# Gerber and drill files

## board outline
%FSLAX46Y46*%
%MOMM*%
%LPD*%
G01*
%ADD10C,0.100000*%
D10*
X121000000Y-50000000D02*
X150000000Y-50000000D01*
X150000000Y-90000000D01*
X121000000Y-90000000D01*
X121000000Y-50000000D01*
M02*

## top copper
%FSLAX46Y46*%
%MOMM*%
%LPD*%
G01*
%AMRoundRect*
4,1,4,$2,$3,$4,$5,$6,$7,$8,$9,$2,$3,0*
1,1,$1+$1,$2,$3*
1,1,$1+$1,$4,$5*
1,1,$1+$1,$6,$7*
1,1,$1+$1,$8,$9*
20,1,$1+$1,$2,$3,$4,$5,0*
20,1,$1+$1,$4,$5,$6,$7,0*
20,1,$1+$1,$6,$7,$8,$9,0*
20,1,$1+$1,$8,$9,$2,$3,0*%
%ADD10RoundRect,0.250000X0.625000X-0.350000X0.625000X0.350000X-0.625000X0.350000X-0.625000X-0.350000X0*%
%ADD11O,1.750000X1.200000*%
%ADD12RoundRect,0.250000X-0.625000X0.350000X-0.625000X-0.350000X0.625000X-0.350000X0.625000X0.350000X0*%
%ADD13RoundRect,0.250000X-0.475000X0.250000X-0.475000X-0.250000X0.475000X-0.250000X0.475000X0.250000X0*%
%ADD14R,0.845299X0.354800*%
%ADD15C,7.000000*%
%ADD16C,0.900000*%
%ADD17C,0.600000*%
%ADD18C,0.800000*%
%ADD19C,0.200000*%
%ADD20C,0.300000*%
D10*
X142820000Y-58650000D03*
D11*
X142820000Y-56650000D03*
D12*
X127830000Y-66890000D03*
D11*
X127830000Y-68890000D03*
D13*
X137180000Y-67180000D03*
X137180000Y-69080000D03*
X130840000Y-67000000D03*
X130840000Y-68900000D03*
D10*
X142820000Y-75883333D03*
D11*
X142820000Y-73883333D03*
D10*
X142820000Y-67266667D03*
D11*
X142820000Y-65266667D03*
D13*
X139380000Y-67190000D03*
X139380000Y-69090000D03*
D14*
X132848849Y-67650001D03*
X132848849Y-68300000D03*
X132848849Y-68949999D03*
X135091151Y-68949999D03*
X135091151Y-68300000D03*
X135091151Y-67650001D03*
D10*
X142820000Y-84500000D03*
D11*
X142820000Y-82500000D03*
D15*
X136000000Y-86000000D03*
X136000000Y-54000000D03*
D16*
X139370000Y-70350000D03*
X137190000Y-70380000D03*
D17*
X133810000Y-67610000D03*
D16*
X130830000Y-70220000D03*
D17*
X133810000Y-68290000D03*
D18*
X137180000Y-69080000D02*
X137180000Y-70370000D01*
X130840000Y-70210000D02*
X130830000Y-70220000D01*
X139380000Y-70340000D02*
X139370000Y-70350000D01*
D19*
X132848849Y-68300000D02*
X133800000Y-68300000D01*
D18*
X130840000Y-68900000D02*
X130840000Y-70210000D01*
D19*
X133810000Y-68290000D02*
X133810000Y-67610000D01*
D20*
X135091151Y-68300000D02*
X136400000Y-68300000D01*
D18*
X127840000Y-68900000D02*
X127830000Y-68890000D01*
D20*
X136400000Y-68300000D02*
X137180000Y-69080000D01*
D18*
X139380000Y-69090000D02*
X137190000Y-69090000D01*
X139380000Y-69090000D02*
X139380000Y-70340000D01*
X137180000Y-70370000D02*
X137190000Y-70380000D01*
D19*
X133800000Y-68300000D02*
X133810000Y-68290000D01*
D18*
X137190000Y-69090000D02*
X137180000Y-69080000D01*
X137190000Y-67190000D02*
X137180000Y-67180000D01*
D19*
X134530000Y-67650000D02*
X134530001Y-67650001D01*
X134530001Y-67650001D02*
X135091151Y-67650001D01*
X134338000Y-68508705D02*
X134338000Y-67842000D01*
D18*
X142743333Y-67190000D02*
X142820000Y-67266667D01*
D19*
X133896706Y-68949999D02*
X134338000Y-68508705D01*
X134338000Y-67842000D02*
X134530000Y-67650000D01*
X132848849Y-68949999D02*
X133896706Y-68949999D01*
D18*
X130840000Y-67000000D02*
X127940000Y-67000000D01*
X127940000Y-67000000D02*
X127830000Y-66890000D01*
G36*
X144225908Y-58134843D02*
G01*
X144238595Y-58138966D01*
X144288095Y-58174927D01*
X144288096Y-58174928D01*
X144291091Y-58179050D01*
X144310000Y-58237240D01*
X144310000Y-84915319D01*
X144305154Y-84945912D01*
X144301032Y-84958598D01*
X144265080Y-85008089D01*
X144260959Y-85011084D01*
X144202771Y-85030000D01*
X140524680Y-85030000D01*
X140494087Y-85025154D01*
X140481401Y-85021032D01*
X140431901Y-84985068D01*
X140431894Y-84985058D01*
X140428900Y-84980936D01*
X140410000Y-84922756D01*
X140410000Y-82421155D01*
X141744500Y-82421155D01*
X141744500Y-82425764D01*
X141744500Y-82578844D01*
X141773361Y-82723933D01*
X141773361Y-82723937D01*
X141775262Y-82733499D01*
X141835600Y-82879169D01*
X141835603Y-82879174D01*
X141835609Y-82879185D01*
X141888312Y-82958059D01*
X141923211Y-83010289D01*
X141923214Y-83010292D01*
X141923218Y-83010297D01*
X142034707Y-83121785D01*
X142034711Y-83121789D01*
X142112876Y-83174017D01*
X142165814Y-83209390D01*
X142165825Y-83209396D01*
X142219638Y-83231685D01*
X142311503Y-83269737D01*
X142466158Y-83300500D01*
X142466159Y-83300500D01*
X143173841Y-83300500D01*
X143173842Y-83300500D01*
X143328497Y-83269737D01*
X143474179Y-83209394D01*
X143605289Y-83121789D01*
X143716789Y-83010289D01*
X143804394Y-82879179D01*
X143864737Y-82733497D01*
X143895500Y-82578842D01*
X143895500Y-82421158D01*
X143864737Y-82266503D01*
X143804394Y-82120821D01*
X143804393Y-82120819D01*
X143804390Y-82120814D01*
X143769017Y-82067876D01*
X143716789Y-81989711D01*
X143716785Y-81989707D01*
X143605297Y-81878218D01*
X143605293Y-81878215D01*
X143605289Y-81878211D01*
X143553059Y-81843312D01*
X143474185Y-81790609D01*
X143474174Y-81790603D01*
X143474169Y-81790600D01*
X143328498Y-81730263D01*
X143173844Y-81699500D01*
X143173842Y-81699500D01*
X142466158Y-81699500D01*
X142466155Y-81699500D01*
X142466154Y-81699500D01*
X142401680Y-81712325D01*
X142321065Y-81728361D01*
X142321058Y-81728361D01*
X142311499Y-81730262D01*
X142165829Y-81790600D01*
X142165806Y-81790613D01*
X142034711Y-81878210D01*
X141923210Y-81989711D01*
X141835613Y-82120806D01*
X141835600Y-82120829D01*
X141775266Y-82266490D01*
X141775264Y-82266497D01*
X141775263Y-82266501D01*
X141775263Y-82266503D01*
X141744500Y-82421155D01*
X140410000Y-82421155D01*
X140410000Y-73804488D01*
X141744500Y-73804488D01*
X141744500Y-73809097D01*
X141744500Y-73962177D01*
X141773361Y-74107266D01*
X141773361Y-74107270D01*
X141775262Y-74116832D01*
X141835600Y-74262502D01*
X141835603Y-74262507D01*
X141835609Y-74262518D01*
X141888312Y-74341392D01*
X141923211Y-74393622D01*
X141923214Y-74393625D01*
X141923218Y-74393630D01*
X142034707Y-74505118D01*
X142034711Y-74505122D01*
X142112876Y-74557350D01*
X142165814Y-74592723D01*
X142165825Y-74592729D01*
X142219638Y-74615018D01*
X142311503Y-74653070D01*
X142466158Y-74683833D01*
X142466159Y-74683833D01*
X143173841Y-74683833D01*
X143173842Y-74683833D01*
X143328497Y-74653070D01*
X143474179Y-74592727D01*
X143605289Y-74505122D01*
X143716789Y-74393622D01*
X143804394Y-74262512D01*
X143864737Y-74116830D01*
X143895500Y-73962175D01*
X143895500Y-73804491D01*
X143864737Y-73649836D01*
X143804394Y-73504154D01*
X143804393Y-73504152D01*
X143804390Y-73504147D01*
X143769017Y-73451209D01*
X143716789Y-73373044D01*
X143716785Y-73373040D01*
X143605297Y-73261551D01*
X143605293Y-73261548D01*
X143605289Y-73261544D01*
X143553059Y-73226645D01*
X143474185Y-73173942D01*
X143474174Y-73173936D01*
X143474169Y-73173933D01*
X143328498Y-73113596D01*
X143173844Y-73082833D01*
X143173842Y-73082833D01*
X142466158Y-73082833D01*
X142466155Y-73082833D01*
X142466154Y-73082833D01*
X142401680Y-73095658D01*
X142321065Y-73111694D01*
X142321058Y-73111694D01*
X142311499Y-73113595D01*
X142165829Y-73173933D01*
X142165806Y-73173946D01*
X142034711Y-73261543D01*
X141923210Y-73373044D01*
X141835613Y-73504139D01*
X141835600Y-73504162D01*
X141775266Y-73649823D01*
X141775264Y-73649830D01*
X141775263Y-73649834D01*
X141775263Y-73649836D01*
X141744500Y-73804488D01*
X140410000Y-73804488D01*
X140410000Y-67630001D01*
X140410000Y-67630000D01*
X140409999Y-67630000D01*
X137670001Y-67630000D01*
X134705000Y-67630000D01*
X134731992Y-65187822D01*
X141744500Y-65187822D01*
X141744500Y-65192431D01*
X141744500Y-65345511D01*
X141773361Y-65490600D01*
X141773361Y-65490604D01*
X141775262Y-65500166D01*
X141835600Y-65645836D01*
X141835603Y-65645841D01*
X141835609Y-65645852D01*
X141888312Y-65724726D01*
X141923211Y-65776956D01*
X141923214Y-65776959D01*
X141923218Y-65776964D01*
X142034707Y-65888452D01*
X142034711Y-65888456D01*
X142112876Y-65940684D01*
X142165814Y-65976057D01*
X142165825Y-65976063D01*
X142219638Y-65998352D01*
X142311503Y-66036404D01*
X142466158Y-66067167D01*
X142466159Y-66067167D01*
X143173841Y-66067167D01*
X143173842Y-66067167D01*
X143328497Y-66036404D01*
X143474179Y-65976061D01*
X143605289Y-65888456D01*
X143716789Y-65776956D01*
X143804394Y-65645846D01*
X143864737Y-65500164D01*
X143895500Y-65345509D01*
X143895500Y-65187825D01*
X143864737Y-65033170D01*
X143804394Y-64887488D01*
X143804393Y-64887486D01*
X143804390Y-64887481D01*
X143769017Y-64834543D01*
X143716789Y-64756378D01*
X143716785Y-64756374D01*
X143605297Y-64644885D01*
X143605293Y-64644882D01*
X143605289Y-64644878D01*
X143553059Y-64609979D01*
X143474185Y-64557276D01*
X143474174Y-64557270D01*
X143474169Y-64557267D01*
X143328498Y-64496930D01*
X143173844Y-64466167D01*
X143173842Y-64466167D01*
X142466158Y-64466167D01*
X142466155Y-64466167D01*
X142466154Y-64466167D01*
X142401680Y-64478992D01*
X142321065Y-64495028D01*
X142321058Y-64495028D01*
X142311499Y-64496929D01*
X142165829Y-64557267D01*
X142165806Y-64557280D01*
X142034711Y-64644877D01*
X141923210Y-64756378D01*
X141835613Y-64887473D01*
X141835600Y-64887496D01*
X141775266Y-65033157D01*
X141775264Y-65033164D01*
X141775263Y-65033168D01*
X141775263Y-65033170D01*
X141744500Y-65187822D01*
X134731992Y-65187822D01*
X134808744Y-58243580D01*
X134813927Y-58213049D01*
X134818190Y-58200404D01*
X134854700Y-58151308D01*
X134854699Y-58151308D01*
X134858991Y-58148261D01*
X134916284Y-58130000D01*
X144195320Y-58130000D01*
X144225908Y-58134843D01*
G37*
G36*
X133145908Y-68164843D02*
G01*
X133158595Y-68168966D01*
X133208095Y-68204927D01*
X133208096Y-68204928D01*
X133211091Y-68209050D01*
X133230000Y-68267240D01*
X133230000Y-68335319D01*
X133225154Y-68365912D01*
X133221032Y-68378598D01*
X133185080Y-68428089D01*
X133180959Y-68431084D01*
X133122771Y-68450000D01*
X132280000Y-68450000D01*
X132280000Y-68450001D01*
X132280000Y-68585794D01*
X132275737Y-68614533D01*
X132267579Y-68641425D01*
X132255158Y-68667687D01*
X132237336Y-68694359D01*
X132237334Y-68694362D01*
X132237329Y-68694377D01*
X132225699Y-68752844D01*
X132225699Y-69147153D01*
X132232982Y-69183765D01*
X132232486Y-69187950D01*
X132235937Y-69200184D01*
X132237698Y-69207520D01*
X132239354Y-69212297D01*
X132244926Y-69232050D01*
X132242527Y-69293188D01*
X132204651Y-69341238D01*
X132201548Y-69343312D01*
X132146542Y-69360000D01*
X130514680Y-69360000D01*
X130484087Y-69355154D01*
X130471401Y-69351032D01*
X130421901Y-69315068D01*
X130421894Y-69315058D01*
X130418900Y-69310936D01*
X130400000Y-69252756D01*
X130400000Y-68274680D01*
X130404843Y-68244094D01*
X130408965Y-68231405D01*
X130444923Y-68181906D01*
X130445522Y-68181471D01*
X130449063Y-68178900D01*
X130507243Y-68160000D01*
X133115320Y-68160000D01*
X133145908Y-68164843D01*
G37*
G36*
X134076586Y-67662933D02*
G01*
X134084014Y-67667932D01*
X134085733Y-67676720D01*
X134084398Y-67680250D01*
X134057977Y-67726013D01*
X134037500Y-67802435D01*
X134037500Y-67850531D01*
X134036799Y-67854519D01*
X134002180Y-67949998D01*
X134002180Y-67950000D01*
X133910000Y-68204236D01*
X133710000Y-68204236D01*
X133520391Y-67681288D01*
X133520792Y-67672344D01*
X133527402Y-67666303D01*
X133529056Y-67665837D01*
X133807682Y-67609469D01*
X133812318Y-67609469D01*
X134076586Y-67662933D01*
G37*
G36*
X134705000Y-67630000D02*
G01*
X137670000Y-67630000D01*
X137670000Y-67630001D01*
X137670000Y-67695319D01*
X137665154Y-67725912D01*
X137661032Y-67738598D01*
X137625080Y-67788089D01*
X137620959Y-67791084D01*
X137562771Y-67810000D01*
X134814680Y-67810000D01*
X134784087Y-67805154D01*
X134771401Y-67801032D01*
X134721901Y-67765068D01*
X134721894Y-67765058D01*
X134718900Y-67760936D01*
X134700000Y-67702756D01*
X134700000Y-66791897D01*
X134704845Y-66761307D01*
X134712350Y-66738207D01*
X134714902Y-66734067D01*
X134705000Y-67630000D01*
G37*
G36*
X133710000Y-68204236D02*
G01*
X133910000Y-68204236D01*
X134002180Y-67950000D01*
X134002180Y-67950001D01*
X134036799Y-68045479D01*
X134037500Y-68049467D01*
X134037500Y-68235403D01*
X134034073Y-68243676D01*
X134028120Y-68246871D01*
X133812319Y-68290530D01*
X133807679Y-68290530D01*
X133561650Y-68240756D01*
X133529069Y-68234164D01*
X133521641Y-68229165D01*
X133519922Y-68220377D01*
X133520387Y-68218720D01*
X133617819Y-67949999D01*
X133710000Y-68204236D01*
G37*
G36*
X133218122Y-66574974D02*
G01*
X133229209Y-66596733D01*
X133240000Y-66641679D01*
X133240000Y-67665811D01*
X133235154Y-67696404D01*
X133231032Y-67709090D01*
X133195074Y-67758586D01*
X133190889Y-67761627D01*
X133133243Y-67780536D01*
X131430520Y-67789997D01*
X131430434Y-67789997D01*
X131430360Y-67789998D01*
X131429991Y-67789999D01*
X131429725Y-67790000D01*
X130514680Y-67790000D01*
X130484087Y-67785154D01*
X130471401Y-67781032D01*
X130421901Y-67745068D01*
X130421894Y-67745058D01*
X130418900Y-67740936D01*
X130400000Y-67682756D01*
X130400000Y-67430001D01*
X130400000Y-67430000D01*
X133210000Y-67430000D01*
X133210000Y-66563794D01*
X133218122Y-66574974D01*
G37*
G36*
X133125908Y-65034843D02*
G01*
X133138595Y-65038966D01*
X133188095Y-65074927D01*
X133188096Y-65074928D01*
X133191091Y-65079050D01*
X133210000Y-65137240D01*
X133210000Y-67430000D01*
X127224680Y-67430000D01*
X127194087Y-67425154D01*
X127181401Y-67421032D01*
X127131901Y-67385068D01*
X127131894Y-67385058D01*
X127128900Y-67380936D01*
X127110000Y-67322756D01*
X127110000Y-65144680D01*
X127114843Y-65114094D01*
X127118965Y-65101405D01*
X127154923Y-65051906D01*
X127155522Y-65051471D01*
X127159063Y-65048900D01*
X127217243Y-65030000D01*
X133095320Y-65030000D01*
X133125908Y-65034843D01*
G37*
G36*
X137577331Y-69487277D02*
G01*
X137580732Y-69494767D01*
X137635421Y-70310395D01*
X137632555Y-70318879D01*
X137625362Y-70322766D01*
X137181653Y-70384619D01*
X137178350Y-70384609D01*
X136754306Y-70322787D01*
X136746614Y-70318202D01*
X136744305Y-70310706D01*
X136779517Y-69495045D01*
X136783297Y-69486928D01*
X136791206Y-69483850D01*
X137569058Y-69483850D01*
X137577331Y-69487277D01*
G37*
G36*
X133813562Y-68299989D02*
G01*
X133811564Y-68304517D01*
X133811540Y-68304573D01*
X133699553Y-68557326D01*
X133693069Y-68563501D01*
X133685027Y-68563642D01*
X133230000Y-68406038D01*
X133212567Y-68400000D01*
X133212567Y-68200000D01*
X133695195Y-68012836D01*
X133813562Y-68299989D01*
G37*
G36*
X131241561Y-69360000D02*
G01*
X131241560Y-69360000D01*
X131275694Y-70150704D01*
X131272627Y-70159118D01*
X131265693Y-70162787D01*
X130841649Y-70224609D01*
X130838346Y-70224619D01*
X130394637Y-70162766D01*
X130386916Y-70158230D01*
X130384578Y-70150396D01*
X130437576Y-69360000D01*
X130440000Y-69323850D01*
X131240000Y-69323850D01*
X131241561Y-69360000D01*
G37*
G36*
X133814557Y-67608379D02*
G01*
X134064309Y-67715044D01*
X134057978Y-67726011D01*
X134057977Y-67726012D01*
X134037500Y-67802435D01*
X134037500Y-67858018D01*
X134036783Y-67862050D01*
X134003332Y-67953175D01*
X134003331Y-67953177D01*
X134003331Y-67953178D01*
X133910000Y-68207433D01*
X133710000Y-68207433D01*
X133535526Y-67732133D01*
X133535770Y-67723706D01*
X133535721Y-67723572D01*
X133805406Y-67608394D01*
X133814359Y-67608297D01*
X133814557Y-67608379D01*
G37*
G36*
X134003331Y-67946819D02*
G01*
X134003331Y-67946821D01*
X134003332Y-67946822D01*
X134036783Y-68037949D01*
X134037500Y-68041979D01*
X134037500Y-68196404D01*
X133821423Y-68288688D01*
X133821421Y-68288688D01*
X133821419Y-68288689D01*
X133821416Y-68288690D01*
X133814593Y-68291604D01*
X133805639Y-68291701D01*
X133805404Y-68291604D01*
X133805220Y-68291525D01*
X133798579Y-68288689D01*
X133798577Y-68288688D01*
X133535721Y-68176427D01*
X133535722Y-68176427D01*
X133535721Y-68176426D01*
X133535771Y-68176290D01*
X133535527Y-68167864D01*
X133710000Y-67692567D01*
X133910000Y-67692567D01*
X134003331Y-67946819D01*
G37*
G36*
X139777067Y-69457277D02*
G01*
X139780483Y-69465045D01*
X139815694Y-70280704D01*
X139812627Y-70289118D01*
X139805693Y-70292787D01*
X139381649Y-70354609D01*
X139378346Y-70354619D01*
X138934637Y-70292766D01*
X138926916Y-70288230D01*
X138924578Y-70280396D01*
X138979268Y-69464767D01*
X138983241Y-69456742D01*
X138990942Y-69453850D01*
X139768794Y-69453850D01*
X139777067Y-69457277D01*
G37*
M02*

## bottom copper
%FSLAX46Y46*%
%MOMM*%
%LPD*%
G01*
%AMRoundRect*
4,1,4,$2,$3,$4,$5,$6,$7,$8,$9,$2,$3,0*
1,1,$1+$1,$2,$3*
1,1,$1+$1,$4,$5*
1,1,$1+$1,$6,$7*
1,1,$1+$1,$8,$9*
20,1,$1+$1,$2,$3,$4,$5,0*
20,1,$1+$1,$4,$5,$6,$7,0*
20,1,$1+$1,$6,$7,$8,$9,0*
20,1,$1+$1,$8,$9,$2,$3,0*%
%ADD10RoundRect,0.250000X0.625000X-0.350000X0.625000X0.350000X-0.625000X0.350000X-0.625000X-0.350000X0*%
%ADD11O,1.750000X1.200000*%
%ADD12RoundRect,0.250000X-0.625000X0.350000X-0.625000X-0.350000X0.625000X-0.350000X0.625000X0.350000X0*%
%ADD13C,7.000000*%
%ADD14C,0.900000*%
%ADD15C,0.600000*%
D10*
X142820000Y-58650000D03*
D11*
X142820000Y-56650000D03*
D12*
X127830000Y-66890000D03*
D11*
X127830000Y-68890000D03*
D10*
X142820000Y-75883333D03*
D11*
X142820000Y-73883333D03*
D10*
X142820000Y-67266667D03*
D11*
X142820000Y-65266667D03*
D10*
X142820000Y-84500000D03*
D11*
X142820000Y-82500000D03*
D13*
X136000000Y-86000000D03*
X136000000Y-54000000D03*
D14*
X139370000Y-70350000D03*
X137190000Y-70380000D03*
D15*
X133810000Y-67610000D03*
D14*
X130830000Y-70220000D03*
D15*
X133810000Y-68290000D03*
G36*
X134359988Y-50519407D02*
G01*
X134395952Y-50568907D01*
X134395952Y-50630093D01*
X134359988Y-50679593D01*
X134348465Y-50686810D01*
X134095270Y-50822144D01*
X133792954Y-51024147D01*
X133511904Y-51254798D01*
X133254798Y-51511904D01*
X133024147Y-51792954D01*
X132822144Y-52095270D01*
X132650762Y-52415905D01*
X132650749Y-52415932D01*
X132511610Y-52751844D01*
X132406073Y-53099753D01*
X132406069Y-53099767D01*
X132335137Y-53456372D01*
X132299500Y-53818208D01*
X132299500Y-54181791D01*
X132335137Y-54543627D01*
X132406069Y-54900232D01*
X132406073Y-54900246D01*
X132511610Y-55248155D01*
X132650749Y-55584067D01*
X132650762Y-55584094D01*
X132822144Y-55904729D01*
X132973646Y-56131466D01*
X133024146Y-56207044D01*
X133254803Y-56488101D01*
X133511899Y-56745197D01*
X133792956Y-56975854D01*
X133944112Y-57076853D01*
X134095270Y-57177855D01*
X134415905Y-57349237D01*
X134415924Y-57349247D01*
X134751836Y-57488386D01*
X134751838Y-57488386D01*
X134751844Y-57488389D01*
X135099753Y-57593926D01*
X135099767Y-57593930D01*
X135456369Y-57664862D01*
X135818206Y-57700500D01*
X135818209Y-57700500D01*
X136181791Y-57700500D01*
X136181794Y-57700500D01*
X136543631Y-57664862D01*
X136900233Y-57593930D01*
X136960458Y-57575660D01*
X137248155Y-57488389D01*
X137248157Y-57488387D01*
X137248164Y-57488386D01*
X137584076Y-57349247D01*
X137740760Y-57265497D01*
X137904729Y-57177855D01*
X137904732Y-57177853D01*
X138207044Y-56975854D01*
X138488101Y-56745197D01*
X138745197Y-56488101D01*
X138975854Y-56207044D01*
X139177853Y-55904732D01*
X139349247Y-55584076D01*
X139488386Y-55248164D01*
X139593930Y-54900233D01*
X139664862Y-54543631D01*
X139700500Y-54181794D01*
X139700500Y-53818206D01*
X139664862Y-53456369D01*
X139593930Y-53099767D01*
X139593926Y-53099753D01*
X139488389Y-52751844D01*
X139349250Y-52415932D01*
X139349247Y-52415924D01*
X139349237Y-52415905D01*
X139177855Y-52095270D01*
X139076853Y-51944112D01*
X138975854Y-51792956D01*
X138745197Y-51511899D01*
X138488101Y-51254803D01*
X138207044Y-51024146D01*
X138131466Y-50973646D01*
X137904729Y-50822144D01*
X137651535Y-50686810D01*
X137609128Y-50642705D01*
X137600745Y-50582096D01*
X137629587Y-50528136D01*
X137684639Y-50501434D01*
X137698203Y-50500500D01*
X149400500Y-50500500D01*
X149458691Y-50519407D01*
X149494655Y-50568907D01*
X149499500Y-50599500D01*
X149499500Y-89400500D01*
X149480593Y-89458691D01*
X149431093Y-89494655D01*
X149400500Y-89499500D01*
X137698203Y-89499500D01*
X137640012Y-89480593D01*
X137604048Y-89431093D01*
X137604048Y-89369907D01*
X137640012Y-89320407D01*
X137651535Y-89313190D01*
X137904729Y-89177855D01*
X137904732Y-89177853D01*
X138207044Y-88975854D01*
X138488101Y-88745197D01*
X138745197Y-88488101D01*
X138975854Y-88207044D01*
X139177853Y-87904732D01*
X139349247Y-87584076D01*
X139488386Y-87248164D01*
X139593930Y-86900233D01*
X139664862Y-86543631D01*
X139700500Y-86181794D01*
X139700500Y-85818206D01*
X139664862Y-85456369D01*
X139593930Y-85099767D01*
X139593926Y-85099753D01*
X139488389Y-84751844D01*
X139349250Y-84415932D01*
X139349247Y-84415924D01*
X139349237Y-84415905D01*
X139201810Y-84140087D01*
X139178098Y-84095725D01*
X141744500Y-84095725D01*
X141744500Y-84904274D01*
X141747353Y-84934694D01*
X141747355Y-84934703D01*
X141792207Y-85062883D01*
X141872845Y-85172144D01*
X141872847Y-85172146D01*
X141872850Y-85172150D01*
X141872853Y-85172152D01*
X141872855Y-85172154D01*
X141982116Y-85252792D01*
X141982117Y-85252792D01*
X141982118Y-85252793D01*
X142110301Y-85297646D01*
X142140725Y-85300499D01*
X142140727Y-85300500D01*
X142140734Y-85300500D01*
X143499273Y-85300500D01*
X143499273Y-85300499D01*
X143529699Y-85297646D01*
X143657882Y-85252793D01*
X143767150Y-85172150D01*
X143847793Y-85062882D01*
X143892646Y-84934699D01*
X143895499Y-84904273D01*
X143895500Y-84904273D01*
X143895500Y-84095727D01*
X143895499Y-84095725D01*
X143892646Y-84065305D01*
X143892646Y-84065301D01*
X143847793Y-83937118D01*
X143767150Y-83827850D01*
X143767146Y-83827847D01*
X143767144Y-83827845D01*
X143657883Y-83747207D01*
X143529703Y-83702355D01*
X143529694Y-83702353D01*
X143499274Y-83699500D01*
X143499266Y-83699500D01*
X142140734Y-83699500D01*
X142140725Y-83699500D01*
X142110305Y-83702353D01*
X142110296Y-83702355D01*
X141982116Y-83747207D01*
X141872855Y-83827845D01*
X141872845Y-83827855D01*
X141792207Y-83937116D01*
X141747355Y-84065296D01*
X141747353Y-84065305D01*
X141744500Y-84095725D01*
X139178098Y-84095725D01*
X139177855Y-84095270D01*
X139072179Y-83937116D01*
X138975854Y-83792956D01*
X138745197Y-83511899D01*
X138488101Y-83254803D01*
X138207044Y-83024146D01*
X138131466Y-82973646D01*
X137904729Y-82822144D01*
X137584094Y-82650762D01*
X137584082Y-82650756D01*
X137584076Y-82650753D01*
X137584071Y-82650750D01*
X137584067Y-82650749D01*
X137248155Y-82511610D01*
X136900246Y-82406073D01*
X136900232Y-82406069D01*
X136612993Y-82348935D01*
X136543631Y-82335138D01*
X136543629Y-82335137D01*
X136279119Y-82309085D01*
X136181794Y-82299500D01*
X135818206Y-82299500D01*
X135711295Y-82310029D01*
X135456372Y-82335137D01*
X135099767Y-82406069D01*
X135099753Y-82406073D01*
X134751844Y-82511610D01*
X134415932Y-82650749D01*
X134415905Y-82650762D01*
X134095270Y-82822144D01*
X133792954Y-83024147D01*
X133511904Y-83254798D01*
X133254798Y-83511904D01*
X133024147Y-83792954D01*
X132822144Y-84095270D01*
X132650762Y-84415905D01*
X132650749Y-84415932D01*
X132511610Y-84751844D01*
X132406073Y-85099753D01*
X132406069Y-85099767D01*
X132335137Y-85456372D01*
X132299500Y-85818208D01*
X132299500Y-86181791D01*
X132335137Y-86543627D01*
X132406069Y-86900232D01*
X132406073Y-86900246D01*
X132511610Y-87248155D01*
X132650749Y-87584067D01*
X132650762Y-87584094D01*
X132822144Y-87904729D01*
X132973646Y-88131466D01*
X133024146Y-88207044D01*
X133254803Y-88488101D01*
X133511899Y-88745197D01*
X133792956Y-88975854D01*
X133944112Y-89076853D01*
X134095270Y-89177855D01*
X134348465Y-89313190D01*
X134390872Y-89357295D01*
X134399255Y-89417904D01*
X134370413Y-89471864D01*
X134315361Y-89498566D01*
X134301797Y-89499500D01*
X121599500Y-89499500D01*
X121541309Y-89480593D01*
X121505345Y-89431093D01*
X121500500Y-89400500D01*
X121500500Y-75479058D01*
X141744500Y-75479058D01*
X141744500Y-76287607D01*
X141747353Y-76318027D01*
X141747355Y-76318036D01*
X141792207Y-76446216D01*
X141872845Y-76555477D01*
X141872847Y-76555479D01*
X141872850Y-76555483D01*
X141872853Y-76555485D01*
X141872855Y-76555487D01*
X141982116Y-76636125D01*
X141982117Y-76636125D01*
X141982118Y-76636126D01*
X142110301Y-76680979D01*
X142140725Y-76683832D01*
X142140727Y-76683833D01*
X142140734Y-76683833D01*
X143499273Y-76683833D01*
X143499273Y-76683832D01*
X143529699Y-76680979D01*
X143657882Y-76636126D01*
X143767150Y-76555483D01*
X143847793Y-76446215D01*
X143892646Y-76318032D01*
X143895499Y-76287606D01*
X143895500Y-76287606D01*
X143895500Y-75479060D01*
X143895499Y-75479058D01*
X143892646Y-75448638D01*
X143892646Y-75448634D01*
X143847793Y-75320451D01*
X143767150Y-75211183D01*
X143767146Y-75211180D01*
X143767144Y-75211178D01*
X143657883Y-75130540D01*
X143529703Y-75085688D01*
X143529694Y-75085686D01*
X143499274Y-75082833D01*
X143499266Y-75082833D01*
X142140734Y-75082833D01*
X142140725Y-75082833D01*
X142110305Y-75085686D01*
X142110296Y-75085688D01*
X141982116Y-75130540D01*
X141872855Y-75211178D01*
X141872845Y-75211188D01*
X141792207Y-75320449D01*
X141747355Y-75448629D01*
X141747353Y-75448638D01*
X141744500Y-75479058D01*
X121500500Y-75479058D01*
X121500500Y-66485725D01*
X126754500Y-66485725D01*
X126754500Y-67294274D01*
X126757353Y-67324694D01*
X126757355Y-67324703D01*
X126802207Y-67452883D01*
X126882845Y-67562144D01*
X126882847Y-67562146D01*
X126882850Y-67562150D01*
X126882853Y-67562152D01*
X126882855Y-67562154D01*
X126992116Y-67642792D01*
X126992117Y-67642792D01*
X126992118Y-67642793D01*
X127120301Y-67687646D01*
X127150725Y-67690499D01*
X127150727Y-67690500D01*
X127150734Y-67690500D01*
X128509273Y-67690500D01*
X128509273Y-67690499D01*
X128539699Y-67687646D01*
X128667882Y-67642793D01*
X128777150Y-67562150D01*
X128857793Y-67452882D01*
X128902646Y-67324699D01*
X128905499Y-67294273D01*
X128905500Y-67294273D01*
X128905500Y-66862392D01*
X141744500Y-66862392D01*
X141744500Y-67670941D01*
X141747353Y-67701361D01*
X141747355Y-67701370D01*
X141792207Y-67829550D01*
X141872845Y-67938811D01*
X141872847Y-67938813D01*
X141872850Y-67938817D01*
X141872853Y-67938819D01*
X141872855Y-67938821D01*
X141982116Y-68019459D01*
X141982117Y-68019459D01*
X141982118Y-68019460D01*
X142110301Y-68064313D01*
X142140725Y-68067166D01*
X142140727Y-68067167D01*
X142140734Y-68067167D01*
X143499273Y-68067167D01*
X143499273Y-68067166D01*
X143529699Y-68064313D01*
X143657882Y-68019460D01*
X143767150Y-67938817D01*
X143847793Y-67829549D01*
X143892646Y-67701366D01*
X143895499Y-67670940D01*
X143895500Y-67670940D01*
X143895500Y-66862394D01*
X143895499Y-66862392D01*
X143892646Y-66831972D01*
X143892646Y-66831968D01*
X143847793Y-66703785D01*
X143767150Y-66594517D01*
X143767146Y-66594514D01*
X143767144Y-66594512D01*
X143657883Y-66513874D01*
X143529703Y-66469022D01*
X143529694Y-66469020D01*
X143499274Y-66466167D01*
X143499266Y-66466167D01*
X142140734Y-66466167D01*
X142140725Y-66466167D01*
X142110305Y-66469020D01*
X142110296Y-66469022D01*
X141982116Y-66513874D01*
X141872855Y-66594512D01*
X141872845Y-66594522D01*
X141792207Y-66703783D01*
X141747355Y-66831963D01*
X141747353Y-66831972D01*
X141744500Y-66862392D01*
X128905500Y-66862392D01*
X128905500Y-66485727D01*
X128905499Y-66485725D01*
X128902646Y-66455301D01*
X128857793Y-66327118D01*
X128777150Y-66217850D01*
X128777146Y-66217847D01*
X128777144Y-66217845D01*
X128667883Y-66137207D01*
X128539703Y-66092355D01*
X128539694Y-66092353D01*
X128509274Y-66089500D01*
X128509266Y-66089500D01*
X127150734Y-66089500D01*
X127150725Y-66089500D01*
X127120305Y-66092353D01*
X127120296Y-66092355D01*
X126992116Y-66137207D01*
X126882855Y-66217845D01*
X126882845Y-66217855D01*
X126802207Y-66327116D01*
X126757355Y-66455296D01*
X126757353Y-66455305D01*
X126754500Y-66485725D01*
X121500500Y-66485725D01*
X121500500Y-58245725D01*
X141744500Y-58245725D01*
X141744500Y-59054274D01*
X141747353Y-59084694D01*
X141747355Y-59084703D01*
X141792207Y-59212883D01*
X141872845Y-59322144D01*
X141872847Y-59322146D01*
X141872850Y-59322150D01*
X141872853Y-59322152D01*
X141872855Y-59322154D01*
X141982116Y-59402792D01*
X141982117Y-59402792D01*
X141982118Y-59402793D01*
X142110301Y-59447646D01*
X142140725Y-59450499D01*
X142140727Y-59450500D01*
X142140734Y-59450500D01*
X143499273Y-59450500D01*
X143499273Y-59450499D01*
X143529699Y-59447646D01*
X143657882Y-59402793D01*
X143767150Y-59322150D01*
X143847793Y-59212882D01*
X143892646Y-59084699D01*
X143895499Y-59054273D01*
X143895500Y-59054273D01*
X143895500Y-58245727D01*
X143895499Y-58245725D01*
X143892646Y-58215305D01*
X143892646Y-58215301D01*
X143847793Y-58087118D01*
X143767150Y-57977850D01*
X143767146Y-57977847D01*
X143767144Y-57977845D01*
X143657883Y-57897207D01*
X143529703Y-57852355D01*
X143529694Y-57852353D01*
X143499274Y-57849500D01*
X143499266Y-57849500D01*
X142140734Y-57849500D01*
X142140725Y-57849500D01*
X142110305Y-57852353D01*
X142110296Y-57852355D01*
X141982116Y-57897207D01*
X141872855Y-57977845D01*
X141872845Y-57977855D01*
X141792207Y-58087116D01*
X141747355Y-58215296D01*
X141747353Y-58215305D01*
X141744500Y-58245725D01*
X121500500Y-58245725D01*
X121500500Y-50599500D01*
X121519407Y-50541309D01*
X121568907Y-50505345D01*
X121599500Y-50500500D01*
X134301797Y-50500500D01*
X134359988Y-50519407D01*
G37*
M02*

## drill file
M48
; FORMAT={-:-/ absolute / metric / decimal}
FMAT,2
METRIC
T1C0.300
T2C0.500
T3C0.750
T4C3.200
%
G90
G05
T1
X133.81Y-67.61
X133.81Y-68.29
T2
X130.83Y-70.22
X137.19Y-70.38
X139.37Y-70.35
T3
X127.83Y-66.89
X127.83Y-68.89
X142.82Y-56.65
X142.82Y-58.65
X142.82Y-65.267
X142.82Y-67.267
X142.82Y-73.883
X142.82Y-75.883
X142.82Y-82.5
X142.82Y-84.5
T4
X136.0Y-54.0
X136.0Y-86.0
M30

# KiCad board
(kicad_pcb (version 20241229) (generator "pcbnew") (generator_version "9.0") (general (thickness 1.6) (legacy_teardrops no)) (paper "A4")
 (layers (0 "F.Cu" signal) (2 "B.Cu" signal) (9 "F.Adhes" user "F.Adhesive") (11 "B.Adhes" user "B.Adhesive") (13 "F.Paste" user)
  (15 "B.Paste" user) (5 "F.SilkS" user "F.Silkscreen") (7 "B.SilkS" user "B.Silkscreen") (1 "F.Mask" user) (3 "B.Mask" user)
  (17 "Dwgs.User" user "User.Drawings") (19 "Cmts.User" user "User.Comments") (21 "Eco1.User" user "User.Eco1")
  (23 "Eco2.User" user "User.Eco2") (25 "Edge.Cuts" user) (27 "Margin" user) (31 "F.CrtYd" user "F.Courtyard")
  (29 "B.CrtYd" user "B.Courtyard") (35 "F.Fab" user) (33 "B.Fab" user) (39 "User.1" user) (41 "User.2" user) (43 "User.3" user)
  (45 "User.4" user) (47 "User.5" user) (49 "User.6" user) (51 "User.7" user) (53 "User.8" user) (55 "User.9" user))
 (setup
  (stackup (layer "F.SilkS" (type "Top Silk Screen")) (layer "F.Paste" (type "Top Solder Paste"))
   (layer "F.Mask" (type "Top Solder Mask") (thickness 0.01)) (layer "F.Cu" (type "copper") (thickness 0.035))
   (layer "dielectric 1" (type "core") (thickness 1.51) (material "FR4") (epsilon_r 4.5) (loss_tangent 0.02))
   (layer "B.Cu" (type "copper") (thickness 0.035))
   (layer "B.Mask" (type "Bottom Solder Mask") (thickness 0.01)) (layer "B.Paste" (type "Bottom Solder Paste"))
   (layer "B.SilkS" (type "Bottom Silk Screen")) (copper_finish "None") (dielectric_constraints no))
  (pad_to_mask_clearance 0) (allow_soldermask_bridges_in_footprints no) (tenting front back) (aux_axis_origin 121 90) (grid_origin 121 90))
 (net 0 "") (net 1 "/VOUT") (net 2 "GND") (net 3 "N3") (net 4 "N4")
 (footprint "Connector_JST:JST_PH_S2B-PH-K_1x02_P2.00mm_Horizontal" (layer "F.Cu") (at 142.82 58.65 90)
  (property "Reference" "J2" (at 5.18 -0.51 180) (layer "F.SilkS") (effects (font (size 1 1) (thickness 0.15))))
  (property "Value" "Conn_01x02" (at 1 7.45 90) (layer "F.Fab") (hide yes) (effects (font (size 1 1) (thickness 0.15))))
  (pad "1" thru_hole roundrect (at 0 0 90) (size 1.2 1.75) (drill 0.75) (layers "*.Cu" "*.Mask") (remove_unused_layers no)
   (roundrect_rratio 0.208333) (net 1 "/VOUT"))
  (pad "2" thru_hole oval (at 2 0 90) (size 1.2 1.75) (drill 0.75) (layers "*.Cu" "*.Mask") (remove_unused_layers no) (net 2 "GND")))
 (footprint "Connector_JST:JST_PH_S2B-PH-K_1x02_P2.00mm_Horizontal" (layer "F.Cu") (at 127.83 66.89 -90)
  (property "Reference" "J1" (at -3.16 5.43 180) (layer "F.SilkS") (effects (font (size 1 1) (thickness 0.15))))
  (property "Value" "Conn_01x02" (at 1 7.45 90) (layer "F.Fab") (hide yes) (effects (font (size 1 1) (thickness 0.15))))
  (pad "1" thru_hole roundrect (at 0 0 270) (size 1.2 1.75) (drill 0.75) (layers "*.Cu" "*.Mask") (remove_unused_layers no)
   (roundrect_rratio 0.208333) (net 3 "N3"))
  (pad "2" thru_hole oval (at 2 0 270) (size 1.2 1.75) (drill 0.75) (layers "*.Cu" "*.Mask") (remove_unused_layers no) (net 2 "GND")))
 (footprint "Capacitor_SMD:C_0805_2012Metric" (layer "F.Cu") (at 137.18 68.13 -90)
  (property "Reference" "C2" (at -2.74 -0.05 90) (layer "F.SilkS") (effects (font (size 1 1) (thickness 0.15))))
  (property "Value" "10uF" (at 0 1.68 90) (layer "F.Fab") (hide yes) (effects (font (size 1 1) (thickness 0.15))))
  (pad "1" smd roundrect (at -0.95 0 270) (size 1 1.45) (layers "F.Cu" "F.Mask" "F.Paste") (roundrect_rratio 0.25) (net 1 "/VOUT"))
  (pad "2" smd roundrect (at 0.95 0 270) (size 1 1.45) (layers "F.Cu" "F.Mask" "F.Paste") (roundrect_rratio 0.25) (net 2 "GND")))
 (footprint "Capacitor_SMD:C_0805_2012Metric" (layer "F.Cu") (at 130.84 67.95 -90)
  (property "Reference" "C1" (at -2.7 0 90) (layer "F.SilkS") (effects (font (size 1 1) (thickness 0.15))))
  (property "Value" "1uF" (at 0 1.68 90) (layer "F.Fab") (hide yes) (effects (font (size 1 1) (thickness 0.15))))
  (pad "1" smd roundrect (at -0.95 0 270) (size 1 1.45) (layers "F.Cu" "F.Mask" "F.Paste") (roundrect_rratio 0.25) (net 3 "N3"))
  (pad "2" smd roundrect (at 0.95 0 270) (size 1 1.45) (layers "F.Cu" "F.Mask" "F.Paste") (roundrect_rratio 0.25) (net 2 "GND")))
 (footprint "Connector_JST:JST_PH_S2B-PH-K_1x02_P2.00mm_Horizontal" (layer "F.Cu") (at 142.82 75.883333 90)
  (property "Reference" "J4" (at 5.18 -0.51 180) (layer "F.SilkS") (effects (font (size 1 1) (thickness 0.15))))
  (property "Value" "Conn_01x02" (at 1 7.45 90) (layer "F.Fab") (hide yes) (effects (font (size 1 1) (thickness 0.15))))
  (pad "1" thru_hole roundrect (at 0 0 90) (size 1.2 1.75) (drill 0.75) (layers "*.Cu" "*.Mask") (remove_unused_layers no)
   (roundrect_rratio 0.208333) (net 1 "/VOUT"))
  (pad "2" thru_hole oval (at 2 0 90) (size 1.2 1.75) (drill 0.75) (layers "*.Cu" "*.Mask") (remove_unused_layers no) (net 2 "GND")))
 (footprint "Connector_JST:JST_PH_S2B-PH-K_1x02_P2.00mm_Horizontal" (layer "F.Cu") (at 142.82 67.266667 90)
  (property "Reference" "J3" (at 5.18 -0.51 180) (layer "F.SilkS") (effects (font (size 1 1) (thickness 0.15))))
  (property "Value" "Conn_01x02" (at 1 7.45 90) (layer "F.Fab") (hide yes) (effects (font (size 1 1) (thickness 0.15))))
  (pad "1" thru_hole roundrect (at 0 0 90) (size 1.2 1.75) (drill 0.75) (layers "*.Cu" "*.Mask") (remove_unused_layers no)
   (roundrect_rratio 0.208333) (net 1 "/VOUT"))
  (pad "2" thru_hole oval (at 2 0 90) (size 1.2 1.75) (drill 0.75) (layers "*.Cu" "*.Mask") (remove_unused_layers no) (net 2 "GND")))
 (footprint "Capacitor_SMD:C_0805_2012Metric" (layer "F.Cu") (at 139.38 68.14 -90)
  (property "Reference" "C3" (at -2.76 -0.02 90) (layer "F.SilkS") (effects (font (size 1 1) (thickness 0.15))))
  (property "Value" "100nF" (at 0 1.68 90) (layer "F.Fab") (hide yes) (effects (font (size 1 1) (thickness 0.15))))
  (pad "1" smd roundrect (at -0.95 0 270) (size 1 1.45) (layers "F.Cu" "F.Mask" "F.Paste") (roundrect_rratio 0.25) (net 1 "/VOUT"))
  (pad "2" smd roundrect (at 0.95 0 270) (size 1 1.45) (layers "F.Cu" "F.Mask" "F.Paste") (roundrect_rratio 0.25) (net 2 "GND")))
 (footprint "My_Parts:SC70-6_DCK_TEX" (layer "F.Cu") (at 133.97 68.3)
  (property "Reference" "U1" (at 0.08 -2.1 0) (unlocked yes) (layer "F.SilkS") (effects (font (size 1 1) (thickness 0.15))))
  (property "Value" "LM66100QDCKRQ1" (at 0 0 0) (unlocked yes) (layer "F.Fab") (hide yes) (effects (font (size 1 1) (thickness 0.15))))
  (pad "1" smd rect (at -1.121151 -0.649999) (size 0.845299 0.3548) (layers "F.Cu" "F.Mask" "F.Paste") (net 3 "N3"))
  (pad "2" smd rect (at -1.121151 0) (size 0.845299 0.3548) (layers "F.Cu" "F.Mask" "F.Paste") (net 2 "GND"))
  (pad "3" smd rect (at -1.121151 0.649999) (size 0.845299 0.3548) (layers "F.Cu" "F.Mask" "F.Paste") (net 1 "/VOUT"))
  (pad "4" smd rect (at 1.121151 0.649999) (size 0.845299 0.3548) (layers "F.Cu" "F.Mask" "F.Paste") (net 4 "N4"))
  (pad "5" smd rect (at 1.121151 0) (size 0.845299 0.3548) (layers "F.Cu" "F.Mask" "F.Paste") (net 2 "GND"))
  (pad "6" smd rect (at 1.121151 -0.649999) (size 0.845299 0.3548) (layers "F.Cu" "F.Mask" "F.Paste") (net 1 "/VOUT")))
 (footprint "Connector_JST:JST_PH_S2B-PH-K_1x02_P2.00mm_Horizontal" (layer "F.Cu") (at 142.82 84.5 90)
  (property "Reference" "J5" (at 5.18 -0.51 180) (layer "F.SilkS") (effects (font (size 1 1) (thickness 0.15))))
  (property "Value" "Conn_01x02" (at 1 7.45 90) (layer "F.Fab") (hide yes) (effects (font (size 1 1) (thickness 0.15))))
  (pad "1" thru_hole roundrect (at 0 0 90) (size 1.2 1.75) (drill 0.75) (layers "*.Cu" "*.Mask") (remove_unused_layers no)
   (roundrect_rratio 0.208333) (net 1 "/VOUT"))
  (pad "2" thru_hole oval (at 2 0 90) (size 1.2 1.75) (drill 0.75) (layers "*.Cu" "*.Mask") (remove_unused_layers no) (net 2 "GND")))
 (gr_rect (start 121 50) (end 150 90) (stroke (width 0.1) (type solid)) (fill no) (layer "Edge.Cuts"))
 (via (at 136 86) (size 7) (drill 3.2) (layers "F.Cu" "B.Cu") (tenting none)
  (teardrops (best_length_ratio 0.5) (max_length 1) (best_width_ratio 1) (max_width 2) (curved_edges no) (filter_ratio 0.9) (enabled yes)
   (allow_two_segments yes) (prefer_zone_connections yes))
  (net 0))
 (via (at 136 54) (size 7) (drill 3.2) (layers "F.Cu" "B.Cu") (tenting none)
  (teardrops (best_length_ratio 0.5) (max_length 1) (best_width_ratio 1) (max_width 2) (curved_edges no) (filter_ratio 0.9) (enabled yes)
   (allow_two_segments yes) (prefer_zone_connections yes))
  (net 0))
 (segment (start 137.18 69.08) (end 137.18 70.37) (width 0.8) (layer "F.Cu") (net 2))
 (segment (start 130.84 70.21) (end 130.83 70.22) (width 0.8) (layer "F.Cu") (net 2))
 (segment (start 139.38 70.34) (end 139.37 70.35) (width 0.8) (layer "F.Cu") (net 2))
 (segment (start 132.848849 68.3) (end 133.8 68.3) (width 0.2) (layer "F.Cu") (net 2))
 (segment (start 130.84 68.9) (end 130.84 70.21) (width 0.8) (layer "F.Cu") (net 2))
 (segment (start 133.81 68.29) (end 133.81 67.61) (width 0.2) (layer "F.Cu") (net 2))
 (segment (start 135.091151 68.3) (end 136.4 68.3) (width 0.3) (layer "F.Cu") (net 2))
 (segment (start 127.84 68.9) (end 127.83 68.89) (width 0.8) (layer "F.Cu") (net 2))
 (segment (start 136.4 68.3) (end 137.18 69.08) (width 0.3) (layer "F.Cu") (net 2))
 (segment (start 139.38 69.09) (end 137.19 69.09) (width 0.8) (layer "F.Cu") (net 2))
 (segment (start 139.38 69.09) (end 139.38 70.34) (width 0.8) (layer "F.Cu") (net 2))
 (segment (start 137.18 70.37) (end 137.19 70.38) (width 0.8) (layer "F.Cu") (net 2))
 (segment (start 133.8 68.3) (end 133.81 68.29) (width 0.2) (layer "F.Cu") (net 2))
 (segment (start 137.19 69.09) (end 137.18 69.08) (width 0.8) (layer "F.Cu") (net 2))
 (via (at 139.37 70.35) (size 0.9) (drill 0.5) (layers "F.Cu" "B.Cu")
  (teardrops (best_length_ratio 0.5) (max_length 1) (best_width_ratio 1) (max_width 2) (curved_edges no) (filter_ratio 0.9) (enabled yes)
   (allow_two_segments yes) (prefer_zone_connections yes))
  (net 2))
 (via (at 137.19 70.38) (size 0.9) (drill 0.5) (layers "F.Cu" "B.Cu")
  (teardrops (best_length_ratio 0.5) (max_length 1) (best_width_ratio 1) (max_width 2) (curved_edges no) (filter_ratio 0.9) (enabled yes)
   (allow_two_segments yes) (prefer_zone_connections yes))
  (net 2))
 (via (at 133.81 67.61) (size 0.6) (drill 0.3) (layers "F.Cu" "B.Cu")
  (teardrops (best_length_ratio 0.5) (max_length 1) (best_width_ratio 1) (max_width 2) (curved_edges no) (filter_ratio 0.9) (enabled yes)
   (allow_two_segments yes) (prefer_zone_connections yes))
  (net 2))
 (via (at 130.83 70.22) (size 0.9) (drill 0.5) (layers "F.Cu" "B.Cu")
  (teardrops (best_length_ratio 0.5) (max_length 1) (best_width_ratio 1) (max_width 2) (curved_edges no) (filter_ratio 0.9) (enabled yes)
   (allow_two_segments yes) (prefer_zone_connections yes))
  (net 2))
 (via (at 133.81 68.29) (size 0.6) (drill 0.3) (layers "F.Cu" "B.Cu")
  (teardrops (best_length_ratio 0.5) (max_length 1) (best_width_ratio 1) (max_width 2) (curved_edges no) (filter_ratio 0.9) (enabled yes)
   (allow_two_segments yes) (prefer_zone_connections yes))
  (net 2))
 (segment (start 137.19 67.19) (end 137.18 67.18) (width 0.8) (layer "F.Cu") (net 1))
 (segment (start 134.53 67.65) (end 134.530001 67.650001) (width 0.2) (layer "F.Cu") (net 1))
 (segment (start 134.530001 67.650001) (end 135.091151 67.650001) (width 0.2) (layer "F.Cu") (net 1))
 (segment (start 134.338 68.508705) (end 134.338 67.842) (width 0.2) (layer "F.Cu") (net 1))
 (segment (start 142.743333 67.19) (end 142.82 67.266667) (width 0.8) (layer "F.Cu") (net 1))
 (segment (start 133.896706 68.949999) (end 134.338 68.508705) (width 0.2) (layer "F.Cu") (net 1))
 (segment (start 134.338 67.842) (end 134.53 67.65) (width 0.2) (layer "F.Cu") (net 1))
 (segment (start 132.848849 68.949999) (end 133.896706 68.949999) (width 0.2) (layer "F.Cu") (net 1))
 (segment (start 130.84 67) (end 127.94 67) (width 0.8) (layer "F.Cu") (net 3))
 (segment (start 127.94 67) (end 127.83 66.89) (width 0.8) (layer "F.Cu") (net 3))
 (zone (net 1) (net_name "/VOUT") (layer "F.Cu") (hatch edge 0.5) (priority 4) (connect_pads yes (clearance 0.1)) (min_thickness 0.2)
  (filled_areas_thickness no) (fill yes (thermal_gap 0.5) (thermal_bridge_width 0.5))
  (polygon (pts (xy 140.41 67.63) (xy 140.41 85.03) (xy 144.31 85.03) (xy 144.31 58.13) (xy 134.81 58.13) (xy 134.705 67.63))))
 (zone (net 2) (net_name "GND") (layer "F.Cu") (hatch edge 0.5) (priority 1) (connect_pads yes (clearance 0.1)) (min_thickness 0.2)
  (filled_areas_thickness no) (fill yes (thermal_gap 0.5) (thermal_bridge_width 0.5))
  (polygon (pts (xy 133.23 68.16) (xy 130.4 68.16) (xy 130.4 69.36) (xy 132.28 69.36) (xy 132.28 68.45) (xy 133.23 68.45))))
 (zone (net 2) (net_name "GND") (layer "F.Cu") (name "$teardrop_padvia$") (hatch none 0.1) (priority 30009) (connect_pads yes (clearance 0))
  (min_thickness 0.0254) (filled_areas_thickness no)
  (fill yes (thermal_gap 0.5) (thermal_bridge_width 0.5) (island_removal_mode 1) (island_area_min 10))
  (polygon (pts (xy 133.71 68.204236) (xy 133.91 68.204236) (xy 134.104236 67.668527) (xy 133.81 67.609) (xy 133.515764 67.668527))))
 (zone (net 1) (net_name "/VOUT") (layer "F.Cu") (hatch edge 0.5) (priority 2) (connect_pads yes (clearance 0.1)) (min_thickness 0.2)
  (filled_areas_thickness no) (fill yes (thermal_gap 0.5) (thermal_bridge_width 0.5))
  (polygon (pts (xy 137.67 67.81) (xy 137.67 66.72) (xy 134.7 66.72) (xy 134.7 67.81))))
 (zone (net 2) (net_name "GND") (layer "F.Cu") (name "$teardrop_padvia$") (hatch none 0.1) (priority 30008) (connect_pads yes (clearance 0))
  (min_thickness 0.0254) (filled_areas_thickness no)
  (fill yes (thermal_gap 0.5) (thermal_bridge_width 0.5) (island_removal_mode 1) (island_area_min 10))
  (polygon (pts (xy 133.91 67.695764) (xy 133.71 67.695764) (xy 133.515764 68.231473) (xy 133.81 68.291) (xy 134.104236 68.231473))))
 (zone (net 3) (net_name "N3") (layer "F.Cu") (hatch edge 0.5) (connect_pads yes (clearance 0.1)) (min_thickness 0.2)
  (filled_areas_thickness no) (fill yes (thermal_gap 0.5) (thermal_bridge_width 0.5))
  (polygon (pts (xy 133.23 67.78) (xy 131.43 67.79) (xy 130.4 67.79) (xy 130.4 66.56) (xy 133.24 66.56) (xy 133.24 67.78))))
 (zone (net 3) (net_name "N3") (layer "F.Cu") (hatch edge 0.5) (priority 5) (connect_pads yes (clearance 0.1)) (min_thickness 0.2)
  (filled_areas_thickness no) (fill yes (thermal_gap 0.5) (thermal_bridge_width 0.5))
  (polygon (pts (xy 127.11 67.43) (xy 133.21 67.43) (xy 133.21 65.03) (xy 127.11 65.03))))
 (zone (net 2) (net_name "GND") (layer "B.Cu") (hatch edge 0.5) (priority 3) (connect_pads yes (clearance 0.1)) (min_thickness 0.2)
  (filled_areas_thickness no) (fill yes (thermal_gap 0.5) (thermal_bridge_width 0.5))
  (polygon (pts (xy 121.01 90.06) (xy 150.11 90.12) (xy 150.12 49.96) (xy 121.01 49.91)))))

